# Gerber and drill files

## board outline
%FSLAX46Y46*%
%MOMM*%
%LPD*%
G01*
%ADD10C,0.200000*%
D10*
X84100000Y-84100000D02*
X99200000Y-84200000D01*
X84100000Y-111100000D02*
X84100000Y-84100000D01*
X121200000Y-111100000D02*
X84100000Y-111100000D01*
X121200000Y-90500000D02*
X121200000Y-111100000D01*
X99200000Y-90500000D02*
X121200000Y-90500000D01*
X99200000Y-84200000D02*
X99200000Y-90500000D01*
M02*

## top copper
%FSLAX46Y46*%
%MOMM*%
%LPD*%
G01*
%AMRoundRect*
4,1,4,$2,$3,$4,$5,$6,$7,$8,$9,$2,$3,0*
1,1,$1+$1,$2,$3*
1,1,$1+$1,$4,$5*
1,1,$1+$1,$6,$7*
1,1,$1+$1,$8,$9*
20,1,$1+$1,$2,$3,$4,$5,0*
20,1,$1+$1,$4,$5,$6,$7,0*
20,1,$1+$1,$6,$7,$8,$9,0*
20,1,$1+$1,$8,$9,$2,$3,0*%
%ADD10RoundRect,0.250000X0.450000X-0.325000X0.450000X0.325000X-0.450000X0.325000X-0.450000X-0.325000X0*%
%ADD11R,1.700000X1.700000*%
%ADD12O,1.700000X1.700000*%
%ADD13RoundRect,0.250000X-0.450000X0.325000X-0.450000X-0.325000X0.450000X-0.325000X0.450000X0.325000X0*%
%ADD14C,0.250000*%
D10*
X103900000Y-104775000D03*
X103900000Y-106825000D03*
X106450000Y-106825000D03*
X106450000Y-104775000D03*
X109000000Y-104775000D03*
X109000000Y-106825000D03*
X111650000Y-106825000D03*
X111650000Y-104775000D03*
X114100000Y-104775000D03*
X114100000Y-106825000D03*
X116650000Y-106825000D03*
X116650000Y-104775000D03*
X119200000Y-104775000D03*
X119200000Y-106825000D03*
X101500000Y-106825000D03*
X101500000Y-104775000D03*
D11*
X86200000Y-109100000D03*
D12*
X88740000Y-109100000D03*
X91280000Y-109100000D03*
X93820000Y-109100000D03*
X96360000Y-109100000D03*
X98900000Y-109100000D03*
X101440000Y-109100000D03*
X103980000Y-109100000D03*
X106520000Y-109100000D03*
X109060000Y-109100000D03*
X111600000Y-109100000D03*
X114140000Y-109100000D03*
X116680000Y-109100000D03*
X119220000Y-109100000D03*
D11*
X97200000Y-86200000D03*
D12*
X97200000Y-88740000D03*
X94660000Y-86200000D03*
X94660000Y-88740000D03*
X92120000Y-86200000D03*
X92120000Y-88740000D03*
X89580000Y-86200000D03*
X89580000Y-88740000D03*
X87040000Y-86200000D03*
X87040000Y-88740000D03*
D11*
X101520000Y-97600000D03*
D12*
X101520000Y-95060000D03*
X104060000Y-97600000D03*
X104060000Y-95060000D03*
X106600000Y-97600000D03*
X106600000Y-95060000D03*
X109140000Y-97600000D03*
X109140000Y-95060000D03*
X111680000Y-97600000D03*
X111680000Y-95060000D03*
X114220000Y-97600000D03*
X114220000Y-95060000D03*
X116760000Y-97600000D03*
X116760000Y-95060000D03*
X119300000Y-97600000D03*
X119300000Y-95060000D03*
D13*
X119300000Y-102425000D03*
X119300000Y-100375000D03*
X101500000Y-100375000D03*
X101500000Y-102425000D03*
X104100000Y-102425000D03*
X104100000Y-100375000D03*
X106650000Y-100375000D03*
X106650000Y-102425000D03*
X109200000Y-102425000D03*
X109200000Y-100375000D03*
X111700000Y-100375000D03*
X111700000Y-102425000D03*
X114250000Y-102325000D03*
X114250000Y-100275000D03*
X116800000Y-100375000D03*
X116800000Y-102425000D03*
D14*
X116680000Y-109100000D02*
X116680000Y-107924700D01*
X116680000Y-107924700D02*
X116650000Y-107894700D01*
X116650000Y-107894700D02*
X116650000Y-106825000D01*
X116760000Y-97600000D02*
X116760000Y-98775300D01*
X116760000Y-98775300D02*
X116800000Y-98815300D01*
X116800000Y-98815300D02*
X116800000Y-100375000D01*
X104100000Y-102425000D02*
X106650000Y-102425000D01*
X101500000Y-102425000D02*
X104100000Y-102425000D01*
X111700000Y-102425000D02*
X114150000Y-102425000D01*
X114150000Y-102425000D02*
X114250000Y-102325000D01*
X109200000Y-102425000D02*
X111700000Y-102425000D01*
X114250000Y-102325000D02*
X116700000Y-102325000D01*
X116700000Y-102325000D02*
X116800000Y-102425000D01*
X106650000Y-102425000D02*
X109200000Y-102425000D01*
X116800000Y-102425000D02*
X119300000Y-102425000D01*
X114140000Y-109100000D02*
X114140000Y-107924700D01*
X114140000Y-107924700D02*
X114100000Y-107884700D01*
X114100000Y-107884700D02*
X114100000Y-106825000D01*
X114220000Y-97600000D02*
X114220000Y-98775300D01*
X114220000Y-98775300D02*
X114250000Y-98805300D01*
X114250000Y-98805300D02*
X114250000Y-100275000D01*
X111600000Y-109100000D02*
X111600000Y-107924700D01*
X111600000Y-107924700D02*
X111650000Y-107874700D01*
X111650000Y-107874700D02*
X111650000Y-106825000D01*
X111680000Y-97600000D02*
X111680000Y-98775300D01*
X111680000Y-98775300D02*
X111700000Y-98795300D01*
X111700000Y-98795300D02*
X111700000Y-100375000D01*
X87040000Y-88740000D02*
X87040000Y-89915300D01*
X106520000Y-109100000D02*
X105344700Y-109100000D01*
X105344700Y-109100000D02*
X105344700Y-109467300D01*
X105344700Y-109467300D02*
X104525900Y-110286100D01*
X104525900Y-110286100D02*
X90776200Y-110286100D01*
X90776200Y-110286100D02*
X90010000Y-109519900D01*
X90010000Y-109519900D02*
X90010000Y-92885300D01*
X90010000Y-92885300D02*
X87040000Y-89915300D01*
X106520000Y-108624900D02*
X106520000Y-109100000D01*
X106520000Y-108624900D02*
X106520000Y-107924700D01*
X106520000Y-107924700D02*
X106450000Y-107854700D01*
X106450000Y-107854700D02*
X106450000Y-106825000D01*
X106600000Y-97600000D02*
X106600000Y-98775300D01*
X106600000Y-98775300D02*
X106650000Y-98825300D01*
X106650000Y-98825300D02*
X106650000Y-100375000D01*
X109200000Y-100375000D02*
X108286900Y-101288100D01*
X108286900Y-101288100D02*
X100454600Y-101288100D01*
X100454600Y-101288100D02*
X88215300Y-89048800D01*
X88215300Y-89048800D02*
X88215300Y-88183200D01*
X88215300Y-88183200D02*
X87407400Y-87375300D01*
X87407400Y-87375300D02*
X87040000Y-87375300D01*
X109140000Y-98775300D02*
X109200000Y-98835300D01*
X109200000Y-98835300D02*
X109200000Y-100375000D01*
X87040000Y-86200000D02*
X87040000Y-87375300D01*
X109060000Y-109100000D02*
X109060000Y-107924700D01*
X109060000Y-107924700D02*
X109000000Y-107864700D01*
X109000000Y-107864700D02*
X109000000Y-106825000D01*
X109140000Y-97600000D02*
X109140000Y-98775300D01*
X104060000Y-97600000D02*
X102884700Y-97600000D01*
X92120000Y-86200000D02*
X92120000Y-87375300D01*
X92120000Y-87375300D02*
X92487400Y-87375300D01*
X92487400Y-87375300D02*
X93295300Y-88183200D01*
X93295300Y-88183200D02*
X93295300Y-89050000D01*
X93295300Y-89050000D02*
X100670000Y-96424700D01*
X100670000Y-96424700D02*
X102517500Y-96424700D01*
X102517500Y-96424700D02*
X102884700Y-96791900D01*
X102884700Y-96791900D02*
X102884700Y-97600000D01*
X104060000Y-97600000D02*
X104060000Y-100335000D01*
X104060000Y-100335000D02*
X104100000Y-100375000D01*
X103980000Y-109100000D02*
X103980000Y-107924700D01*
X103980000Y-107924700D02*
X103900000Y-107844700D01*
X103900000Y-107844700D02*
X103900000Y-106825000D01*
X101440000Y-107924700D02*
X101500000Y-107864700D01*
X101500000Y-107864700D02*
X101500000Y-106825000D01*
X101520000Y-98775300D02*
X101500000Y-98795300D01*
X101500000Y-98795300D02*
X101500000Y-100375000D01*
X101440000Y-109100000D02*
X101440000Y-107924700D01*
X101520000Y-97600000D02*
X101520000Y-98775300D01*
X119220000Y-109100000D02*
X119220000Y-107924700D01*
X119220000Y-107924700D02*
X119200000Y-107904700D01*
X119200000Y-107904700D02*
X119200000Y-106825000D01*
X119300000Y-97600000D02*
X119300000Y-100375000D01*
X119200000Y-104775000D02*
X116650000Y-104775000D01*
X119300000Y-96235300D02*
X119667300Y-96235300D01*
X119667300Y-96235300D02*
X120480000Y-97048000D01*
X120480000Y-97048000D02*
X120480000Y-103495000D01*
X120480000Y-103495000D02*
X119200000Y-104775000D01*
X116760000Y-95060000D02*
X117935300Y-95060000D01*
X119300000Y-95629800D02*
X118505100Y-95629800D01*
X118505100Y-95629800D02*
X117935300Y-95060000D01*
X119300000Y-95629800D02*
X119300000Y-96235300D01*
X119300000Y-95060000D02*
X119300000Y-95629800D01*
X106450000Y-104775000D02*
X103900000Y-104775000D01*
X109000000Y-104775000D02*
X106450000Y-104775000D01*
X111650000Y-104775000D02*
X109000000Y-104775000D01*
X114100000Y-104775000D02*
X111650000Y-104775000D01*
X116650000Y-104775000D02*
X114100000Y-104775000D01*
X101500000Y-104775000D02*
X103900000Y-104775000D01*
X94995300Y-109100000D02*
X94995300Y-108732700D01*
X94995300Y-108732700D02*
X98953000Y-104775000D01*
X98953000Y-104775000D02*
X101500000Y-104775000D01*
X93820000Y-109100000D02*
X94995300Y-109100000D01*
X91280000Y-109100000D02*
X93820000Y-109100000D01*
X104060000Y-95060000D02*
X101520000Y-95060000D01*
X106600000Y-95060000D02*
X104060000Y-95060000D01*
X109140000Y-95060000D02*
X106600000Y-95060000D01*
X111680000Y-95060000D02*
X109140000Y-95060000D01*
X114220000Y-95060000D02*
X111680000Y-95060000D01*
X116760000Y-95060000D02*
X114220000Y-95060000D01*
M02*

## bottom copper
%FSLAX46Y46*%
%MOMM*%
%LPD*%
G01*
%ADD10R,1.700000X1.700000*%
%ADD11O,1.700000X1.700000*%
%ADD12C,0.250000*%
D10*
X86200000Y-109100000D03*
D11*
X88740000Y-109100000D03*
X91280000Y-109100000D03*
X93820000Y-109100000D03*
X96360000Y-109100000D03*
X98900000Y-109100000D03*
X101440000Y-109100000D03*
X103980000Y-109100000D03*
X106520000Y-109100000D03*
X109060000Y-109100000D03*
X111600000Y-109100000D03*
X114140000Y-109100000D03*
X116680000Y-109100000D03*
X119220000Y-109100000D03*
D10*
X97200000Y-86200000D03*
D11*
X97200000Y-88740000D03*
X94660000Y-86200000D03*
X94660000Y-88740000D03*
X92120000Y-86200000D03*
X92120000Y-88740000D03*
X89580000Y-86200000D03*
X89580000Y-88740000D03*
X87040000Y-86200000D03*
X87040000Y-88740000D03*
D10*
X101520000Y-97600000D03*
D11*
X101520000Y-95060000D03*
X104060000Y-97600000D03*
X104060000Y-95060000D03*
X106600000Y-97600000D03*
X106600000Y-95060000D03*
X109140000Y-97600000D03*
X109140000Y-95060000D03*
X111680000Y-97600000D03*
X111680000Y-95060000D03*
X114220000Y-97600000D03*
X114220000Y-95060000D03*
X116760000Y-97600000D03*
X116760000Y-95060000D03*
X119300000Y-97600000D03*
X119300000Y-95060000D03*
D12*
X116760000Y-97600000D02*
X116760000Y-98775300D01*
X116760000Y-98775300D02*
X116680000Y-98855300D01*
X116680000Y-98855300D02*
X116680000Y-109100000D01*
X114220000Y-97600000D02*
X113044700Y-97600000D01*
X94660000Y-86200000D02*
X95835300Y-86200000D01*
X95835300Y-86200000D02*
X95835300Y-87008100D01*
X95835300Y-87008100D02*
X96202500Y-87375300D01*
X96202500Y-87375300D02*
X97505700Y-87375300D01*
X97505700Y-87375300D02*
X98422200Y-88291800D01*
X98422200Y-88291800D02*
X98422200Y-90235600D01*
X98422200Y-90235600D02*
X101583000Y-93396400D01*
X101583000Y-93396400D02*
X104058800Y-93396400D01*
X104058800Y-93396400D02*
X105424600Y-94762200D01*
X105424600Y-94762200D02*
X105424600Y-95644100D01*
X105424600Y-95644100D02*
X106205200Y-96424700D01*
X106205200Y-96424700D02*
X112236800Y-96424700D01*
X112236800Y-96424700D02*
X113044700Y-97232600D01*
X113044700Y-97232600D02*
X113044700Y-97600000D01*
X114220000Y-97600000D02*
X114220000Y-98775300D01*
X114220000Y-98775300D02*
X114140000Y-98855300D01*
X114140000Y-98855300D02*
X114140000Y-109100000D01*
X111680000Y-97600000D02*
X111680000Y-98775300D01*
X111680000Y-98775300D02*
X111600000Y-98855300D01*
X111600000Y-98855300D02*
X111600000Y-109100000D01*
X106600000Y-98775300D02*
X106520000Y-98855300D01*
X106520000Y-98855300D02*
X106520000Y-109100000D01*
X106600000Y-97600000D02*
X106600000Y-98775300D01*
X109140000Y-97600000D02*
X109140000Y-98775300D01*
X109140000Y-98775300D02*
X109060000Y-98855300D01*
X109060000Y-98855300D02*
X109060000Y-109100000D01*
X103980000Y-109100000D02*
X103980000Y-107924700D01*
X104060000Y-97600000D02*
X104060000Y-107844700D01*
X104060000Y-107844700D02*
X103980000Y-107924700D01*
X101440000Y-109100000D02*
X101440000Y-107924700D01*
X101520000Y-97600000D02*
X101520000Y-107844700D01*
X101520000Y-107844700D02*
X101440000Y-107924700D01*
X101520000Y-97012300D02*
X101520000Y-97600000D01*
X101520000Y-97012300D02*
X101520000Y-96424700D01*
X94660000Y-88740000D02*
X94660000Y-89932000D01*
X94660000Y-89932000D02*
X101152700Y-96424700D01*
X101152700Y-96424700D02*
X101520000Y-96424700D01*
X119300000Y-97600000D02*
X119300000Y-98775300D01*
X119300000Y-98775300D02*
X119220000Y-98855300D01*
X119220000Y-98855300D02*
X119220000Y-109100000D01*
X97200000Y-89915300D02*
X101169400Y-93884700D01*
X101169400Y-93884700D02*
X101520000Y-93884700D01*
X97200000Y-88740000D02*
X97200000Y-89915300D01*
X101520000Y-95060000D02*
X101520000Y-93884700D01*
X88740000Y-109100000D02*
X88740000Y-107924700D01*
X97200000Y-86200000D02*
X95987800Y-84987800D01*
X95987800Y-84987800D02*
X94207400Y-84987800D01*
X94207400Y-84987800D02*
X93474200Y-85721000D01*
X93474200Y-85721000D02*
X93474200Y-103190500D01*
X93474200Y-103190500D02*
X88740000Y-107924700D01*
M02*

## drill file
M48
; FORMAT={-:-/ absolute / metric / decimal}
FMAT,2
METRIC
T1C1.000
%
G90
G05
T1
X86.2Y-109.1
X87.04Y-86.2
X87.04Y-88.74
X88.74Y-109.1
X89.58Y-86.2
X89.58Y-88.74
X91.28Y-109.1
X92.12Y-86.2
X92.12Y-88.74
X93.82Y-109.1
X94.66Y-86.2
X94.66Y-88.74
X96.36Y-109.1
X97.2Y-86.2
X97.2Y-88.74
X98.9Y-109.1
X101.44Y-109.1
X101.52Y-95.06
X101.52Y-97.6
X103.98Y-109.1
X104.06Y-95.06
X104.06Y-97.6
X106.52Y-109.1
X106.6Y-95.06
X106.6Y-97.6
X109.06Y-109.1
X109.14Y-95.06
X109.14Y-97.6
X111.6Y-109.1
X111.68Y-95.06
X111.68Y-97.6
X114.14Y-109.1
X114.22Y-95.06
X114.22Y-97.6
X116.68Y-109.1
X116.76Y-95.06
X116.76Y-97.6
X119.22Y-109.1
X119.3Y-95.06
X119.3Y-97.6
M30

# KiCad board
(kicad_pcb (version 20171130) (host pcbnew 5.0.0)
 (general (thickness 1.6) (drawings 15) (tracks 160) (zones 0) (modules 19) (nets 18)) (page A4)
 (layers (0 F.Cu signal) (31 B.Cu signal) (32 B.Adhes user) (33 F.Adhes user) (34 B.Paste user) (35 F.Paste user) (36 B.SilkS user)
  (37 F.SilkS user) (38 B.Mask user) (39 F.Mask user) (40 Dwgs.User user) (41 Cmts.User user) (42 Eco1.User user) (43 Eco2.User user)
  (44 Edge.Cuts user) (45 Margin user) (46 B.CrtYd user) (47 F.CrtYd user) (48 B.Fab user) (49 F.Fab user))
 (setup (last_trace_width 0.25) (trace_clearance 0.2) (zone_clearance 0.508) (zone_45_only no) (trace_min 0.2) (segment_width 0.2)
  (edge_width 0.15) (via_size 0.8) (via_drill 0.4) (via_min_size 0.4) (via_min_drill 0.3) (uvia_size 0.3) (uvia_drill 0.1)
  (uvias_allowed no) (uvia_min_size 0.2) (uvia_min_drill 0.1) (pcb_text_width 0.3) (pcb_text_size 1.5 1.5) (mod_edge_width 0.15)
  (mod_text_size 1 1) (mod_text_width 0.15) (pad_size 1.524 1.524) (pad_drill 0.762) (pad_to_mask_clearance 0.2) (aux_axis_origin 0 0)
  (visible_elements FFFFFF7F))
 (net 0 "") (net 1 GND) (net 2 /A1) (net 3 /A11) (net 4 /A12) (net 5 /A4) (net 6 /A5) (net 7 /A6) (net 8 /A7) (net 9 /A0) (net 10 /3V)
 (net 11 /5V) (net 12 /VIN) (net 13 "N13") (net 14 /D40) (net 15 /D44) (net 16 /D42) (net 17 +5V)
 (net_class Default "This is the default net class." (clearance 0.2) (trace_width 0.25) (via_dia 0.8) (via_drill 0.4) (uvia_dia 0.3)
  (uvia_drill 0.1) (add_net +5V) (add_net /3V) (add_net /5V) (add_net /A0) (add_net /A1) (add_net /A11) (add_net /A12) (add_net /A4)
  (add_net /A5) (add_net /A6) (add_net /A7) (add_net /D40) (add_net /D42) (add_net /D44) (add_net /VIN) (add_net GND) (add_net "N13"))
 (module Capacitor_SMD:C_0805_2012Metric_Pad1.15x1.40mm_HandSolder (layer F.Cu) (at 103.9 105.8 90)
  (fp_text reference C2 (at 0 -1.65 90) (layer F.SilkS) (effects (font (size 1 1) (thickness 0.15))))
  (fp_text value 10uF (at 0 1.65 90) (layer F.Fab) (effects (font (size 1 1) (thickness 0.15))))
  (pad 2 smd roundrect (at 1.025 0 90) (size 1.15 1.4) (layers F.Cu F.Paste F.Mask) (roundrect_rratio 0.217391) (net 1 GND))
  (pad 1 smd roundrect (at -1.025 0 90) (size 1.15 1.4) (layers F.Cu F.Paste F.Mask) (roundrect_rratio 0.217391) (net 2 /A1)))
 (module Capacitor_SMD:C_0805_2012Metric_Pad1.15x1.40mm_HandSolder (layer F.Cu) (at 106.45 105.8 90)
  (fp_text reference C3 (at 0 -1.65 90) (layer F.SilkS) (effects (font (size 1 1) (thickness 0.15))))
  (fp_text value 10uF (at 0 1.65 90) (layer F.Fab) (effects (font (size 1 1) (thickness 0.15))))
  (pad 1 smd roundrect (at -1.025 0 90) (size 1.15 1.4) (layers F.Cu F.Paste F.Mask) (roundrect_rratio 0.217391) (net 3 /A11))
  (pad 2 smd roundrect (at 1.025 0 90) (size 1.15 1.4) (layers F.Cu F.Paste F.Mask) (roundrect_rratio 0.217391) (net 1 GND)))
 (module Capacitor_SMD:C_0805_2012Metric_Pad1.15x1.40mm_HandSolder (layer F.Cu) (at 109 105.8 90)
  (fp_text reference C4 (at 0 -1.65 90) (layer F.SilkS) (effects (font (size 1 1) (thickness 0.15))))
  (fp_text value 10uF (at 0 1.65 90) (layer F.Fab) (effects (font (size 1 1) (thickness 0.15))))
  (pad 2 smd roundrect (at 1.025 0 90) (size 1.15 1.4) (layers F.Cu F.Paste F.Mask) (roundrect_rratio 0.217391) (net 1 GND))
  (pad 1 smd roundrect (at -1.025 0 90) (size 1.15 1.4) (layers F.Cu F.Paste F.Mask) (roundrect_rratio 0.217391) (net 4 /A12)))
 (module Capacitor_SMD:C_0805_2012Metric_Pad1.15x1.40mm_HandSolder (layer F.Cu) (at 111.65 105.8 90)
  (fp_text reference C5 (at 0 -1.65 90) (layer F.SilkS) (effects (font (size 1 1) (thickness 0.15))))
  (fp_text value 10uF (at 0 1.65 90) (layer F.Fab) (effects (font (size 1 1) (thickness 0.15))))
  (pad 1 smd roundrect (at -1.025 0 90) (size 1.15 1.4) (layers F.Cu F.Paste F.Mask) (roundrect_rratio 0.217391) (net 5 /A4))
  (pad 2 smd roundrect (at 1.025 0 90) (size 1.15 1.4) (layers F.Cu F.Paste F.Mask) (roundrect_rratio 0.217391) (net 1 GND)))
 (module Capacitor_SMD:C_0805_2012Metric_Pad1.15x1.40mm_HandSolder (layer F.Cu) (at 114.1 105.8 90)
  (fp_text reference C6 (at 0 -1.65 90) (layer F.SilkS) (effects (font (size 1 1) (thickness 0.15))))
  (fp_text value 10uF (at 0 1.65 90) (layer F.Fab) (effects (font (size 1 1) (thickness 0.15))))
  (pad 2 smd roundrect (at 1.025 0 90) (size 1.15 1.4) (layers F.Cu F.Paste F.Mask) (roundrect_rratio 0.217391) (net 1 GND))
  (pad 1 smd roundrect (at -1.025 0 90) (size 1.15 1.4) (layers F.Cu F.Paste F.Mask) (roundrect_rratio 0.217391) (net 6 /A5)))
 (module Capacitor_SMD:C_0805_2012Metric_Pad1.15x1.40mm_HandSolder (layer F.Cu) (at 116.65 105.8 90)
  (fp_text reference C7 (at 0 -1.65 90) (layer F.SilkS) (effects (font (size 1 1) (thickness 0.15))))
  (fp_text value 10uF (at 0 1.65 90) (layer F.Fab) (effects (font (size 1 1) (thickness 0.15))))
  (pad 1 smd roundrect (at -1.025 0 90) (size 1.15 1.4) (layers F.Cu F.Paste F.Mask) (roundrect_rratio 0.217391) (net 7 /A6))
  (pad 2 smd roundrect (at 1.025 0 90) (size 1.15 1.4) (layers F.Cu F.Paste F.Mask) (roundrect_rratio 0.217391) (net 1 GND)))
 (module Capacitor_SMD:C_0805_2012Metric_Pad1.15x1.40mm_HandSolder (layer F.Cu) (at 119.2 105.8 90)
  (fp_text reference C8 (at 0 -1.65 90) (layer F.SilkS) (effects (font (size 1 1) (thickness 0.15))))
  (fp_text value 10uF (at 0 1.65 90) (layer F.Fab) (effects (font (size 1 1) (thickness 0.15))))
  (pad 2 smd roundrect (at 1.025 0 90) (size 1.15 1.4) (layers F.Cu F.Paste F.Mask) (roundrect_rratio 0.217391) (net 1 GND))
  (pad 1 smd roundrect (at -1.025 0 90) (size 1.15 1.4) (layers F.Cu F.Paste F.Mask) (roundrect_rratio 0.217391) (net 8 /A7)))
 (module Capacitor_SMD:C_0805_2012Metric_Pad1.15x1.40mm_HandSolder (layer F.Cu) (at 101.5 105.8 90)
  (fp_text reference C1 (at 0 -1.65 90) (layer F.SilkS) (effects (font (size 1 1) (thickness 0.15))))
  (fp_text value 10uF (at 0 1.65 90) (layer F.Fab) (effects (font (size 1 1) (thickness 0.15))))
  (pad 1 smd roundrect (at -1.025 0 90) (size 1.15 1.4) (layers F.Cu F.Paste F.Mask) (roundrect_rratio 0.217391) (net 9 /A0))
  (pad 2 smd roundrect (at 1.025 0 90) (size 1.15 1.4) (layers F.Cu F.Paste F.Mask) (roundrect_rratio 0.217391) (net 1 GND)))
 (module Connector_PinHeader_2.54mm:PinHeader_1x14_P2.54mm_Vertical (layer F.Cu) (at 86.2 109.1 90)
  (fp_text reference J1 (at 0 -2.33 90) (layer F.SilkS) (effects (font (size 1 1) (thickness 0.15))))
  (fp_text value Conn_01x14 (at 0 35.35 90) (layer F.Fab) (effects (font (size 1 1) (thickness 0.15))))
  (pad 1 thru_hole rect (at 0 0 90) (size 1.7 1.7) (drill 1) (layers *.Cu *.Mask) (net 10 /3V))
  (pad 2 thru_hole oval (at 0 2.54 90) (size 1.7 1.7) (drill 1) (layers *.Cu *.Mask) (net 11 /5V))
  (pad 3 thru_hole oval (at 0 5.08 90) (size 1.7 1.7) (drill 1) (layers *.Cu *.Mask) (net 1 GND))
  (pad 4 thru_hole oval (at 0 7.62 90) (size 1.7 1.7) (drill 1) (layers *.Cu *.Mask) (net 1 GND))
  (pad 5 thru_hole oval (at 0 10.16 90) (size 1.7 1.7) (drill 1) (layers *.Cu *.Mask) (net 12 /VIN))
  (pad 6 thru_hole oval (at 0 12.7 90) (size 1.7 1.7) (drill 1) (layers *.Cu *.Mask) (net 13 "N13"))
  (pad 7 thru_hole oval (at 0 15.24 90) (size 1.7 1.7) (drill 1) (layers *.Cu *.Mask) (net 9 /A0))
  (pad 8 thru_hole oval (at 0 17.78 90) (size 1.7 1.7) (drill 1) (layers *.Cu *.Mask) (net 2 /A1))
  (pad 9 thru_hole oval (at 0 20.32 90) (size 1.7 1.7) (drill 1) (layers *.Cu *.Mask) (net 3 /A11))
  (pad 10 thru_hole oval (at 0 22.86 90) (size 1.7 1.7) (drill 1) (layers *.Cu *.Mask) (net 4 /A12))
  (pad 11 thru_hole oval (at 0 25.4 90) (size 1.7 1.7) (drill 1) (layers *.Cu *.Mask) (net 5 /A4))
  (pad 12 thru_hole oval (at 0 27.94 90) (size 1.7 1.7) (drill 1) (layers *.Cu *.Mask) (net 6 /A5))
  (pad 13 thru_hole oval (at 0 30.48 90) (size 1.7 1.7) (drill 1) (layers *.Cu *.Mask) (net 7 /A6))
  (pad 14 thru_hole oval (at 0 33.02 90) (size 1.7 1.7) (drill 1) (layers *.Cu *.Mask) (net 8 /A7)))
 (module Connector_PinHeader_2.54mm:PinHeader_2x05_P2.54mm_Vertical (layer F.Cu) (at 97.2 86.2 270)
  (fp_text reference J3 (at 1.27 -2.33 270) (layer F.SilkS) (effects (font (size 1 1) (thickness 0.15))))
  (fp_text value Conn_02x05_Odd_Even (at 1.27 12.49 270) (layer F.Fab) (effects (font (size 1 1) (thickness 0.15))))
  (pad 1 thru_hole rect (at 0 0 270) (size 1.7 1.7) (drill 1) (layers *.Cu *.Mask) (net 11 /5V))
  (pad 2 thru_hole oval (at 2.54 0 270) (size 1.7 1.7) (drill 1) (layers *.Cu *.Mask) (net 1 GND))
  (pad 3 thru_hole oval (at 0 2.54 270) (size 1.7 1.7) (drill 1) (layers *.Cu *.Mask) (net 6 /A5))
  (pad 4 thru_hole oval (at 2.54 2.54 270) (size 1.7 1.7) (drill 1) (layers *.Cu *.Mask) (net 9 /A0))
  (pad 5 thru_hole oval (at 0 5.08 270) (size 1.7 1.7) (drill 1) (layers *.Cu *.Mask) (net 2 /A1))
  (pad 6 thru_hole oval (at 2.54 5.08 270) (size 1.7 1.7) (drill 1) (layers *.Cu *.Mask) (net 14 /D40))
  (pad 7 thru_hole oval (at 0 7.62 270) (size 1.7 1.7) (drill 1) (layers *.Cu *.Mask) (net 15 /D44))
  (pad 8 thru_hole oval (at 2.54 7.62 270) (size 1.7 1.7) (drill 1) (layers *.Cu *.Mask) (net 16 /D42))
  (pad 9 thru_hole oval (at 0 10.16 270) (size 1.7 1.7) (drill 1) (layers *.Cu *.Mask) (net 4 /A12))
  (pad 10 thru_hole oval (at 2.54 10.16 270) (size 1.7 1.7) (drill 1) (layers *.Cu *.Mask) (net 3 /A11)))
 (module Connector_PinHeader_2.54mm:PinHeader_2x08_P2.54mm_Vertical (layer F.Cu) (at 101.52 97.6 90)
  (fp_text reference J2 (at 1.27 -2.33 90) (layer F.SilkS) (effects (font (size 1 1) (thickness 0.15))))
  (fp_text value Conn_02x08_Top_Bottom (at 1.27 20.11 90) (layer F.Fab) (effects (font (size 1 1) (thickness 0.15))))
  (pad 1 thru_hole rect (at 0 0 90) (size 1.7 1.7) (drill 1) (layers *.Cu *.Mask) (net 9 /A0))
  (pad 2 thru_hole oval (at 2.54 0 90) (size 1.7 1.7) (drill 1) (layers *.Cu *.Mask) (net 1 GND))
  (pad 3 thru_hole oval (at 0 2.54 90) (size 1.7 1.7) (drill 1) (layers *.Cu *.Mask) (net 2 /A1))
  (pad 4 thru_hole oval (at 2.54 2.54 90) (size 1.7 1.7) (drill 1) (layers *.Cu *.Mask) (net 1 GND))
  (pad 5 thru_hole oval (at 0 5.08 90) (size 1.7 1.7) (drill 1) (layers *.Cu *.Mask) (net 3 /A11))
  (pad 6 thru_hole oval (at 2.54 5.08 90) (size 1.7 1.7) (drill 1) (layers *.Cu *.Mask) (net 1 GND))
  (pad 7 thru_hole oval (at 0 7.62 90) (size 1.7 1.7) (drill 1) (layers *.Cu *.Mask) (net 4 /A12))
  (pad 8 thru_hole oval (at 2.54 7.62 90) (size 1.7 1.7) (drill 1) (layers *.Cu *.Mask) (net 1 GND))
  (pad 9 thru_hole oval (at 0 10.16 90) (size 1.7 1.7) (drill 1) (layers *.Cu *.Mask) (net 5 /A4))
  (pad 10 thru_hole oval (at 2.54 10.16 90) (size 1.7 1.7) (drill 1) (layers *.Cu *.Mask) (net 1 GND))
  (pad 11 thru_hole oval (at 0 12.7 90) (size 1.7 1.7) (drill 1) (layers *.Cu *.Mask) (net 6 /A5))
  (pad 12 thru_hole oval (at 2.54 12.7 90) (size 1.7 1.7) (drill 1) (layers *.Cu *.Mask) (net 1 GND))
  (pad 13 thru_hole oval (at 0 15.24 90) (size 1.7 1.7) (drill 1) (layers *.Cu *.Mask) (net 7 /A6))
  (pad 14 thru_hole oval (at 2.54 15.24 90) (size 1.7 1.7) (drill 1) (layers *.Cu *.Mask) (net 1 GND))
  (pad 15 thru_hole oval (at 0 17.78 90) (size 1.7 1.7) (drill 1) (layers *.Cu *.Mask) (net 8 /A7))
  (pad 16 thru_hole oval (at 2.54 17.78 90) (size 1.7 1.7) (drill 1) (layers *.Cu *.Mask) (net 1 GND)))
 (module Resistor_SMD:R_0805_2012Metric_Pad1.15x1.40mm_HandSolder (layer F.Cu) (at 119.3 101.4 270)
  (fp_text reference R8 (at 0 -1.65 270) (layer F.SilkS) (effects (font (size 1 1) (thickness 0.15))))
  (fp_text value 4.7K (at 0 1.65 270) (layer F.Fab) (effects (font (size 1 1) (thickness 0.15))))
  (pad 2 smd roundrect (at 1.025 0 270) (size 1.15 1.4) (layers F.Cu F.Paste F.Mask) (roundrect_rratio 0.217391) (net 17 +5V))
  (pad 1 smd roundrect (at -1.025 0 270) (size 1.15 1.4) (layers F.Cu F.Paste F.Mask) (roundrect_rratio 0.217391) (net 8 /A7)))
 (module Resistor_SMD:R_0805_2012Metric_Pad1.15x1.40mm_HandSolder (layer F.Cu) (at 101.5 101.4 270)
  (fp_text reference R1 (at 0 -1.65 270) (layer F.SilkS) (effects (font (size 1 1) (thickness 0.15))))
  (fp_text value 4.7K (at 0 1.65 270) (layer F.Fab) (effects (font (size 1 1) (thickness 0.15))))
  (pad 1 smd roundrect (at -1.025 0 270) (size 1.15 1.4) (layers F.Cu F.Paste F.Mask) (roundrect_rratio 0.217391) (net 9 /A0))
  (pad 2 smd roundrect (at 1.025 0 270) (size 1.15 1.4) (layers F.Cu F.Paste F.Mask) (roundrect_rratio 0.217391) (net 17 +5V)))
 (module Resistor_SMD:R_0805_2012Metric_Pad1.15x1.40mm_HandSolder (layer F.Cu) (at 104.1 101.4 270)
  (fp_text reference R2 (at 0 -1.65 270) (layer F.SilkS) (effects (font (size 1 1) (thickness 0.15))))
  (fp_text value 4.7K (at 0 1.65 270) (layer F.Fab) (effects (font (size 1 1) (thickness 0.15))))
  (pad 2 smd roundrect (at 1.025 0 270) (size 1.15 1.4) (layers F.Cu F.Paste F.Mask) (roundrect_rratio 0.217391) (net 17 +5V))
  (pad 1 smd roundrect (at -1.025 0 270) (size 1.15 1.4) (layers F.Cu F.Paste F.Mask) (roundrect_rratio 0.217391) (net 2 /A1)))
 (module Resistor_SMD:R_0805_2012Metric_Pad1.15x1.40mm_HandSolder (layer F.Cu) (at 106.65 101.4 270)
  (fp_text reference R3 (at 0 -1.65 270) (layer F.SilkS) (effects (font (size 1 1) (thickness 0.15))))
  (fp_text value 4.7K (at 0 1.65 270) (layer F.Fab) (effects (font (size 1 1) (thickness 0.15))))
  (pad 1 smd roundrect (at -1.025 0 270) (size 1.15 1.4) (layers F.Cu F.Paste F.Mask) (roundrect_rratio 0.217391) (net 3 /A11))
  (pad 2 smd roundrect (at 1.025 0 270) (size 1.15 1.4) (layers F.Cu F.Paste F.Mask) (roundrect_rratio 0.217391) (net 17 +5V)))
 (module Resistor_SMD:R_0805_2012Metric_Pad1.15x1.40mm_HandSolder (layer F.Cu) (at 109.2 101.4 270)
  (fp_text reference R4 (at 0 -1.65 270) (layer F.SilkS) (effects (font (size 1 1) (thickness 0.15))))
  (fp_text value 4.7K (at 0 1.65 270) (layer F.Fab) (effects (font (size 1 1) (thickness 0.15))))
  (pad 2 smd roundrect (at 1.025 0 270) (size 1.15 1.4) (layers F.Cu F.Paste F.Mask) (roundrect_rratio 0.217391) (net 17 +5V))
  (pad 1 smd roundrect (at -1.025 0 270) (size 1.15 1.4) (layers F.Cu F.Paste F.Mask) (roundrect_rratio 0.217391) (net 4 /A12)))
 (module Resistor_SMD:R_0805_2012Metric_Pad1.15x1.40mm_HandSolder (layer F.Cu) (at 111.7 101.4 270)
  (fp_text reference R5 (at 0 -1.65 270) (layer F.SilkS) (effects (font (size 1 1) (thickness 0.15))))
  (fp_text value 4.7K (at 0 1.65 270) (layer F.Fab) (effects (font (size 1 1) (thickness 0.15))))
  (pad 1 smd roundrect (at -1.025 0 270) (size 1.15 1.4) (layers F.Cu F.Paste F.Mask) (roundrect_rratio 0.217391) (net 5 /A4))
  (pad 2 smd roundrect (at 1.025 0 270) (size 1.15 1.4) (layers F.Cu F.Paste F.Mask) (roundrect_rratio 0.217391) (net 17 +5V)))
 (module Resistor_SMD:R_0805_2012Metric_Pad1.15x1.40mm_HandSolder (layer F.Cu) (at 114.25 101.3 270)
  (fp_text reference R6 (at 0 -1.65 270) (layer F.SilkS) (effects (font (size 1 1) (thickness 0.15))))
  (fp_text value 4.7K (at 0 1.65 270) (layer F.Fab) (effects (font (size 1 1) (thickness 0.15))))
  (pad 2 smd roundrect (at 1.025 0 270) (size 1.15 1.4) (layers F.Cu F.Paste F.Mask) (roundrect_rratio 0.217391) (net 17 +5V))
  (pad 1 smd roundrect (at -1.025 0 270) (size 1.15 1.4) (layers F.Cu F.Paste F.Mask) (roundrect_rratio 0.217391) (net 6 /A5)))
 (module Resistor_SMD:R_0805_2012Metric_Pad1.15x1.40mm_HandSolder (layer F.Cu) (at 116.8 101.4 270)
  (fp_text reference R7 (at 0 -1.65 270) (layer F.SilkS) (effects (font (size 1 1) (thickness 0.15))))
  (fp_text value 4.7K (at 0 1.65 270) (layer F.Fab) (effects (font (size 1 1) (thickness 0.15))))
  (pad 1 smd roundrect (at -1.025 0 270) (size 1.15 1.4) (layers F.Cu F.Paste F.Mask) (roundrect_rratio 0.217391) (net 7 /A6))
  (pad 2 smd roundrect (at 1.025 0 270) (size 1.15 1.4) (layers F.Cu F.Paste F.Mask) (roundrect_rratio 0.217391) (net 17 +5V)))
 (gr_line (start 84.1 84.1) (end 99.2 84.2) (layer Edge.Cuts) (width 0.2))
 (gr_line (start 84.1 111.1) (end 84.1 84.1) (layer Edge.Cuts) (width 0.2))
 (gr_line (start 121.2 111.1) (end 84.1 111.1) (layer Edge.Cuts) (width 0.2))
 (gr_line (start 121.2 90.5) (end 121.2 111.1) (layer Edge.Cuts) (width 0.2))
 (gr_line (start 99.2 90.5) (end 121.2 90.5) (layer Edge.Cuts) (width 0.2))
 (gr_line (start 99.2 84.2) (end 99.2 90.5) (layer Edge.Cuts) (width 0.2))
 (segment (start 116.76 97.6) (end 116.76 98.7753) (width 0.25) (layer B.Cu) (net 7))
 (segment (start 116.76 98.7753) (end 116.68 98.8553) (width 0.25) (layer B.Cu) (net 7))
 (segment (start 116.68 98.8553) (end 116.68 109.1) (width 0.25) (layer B.Cu) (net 7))
 (segment (start 116.68 109.1) (end 116.68 107.9247) (width 0.25) (layer F.Cu) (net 7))
 (segment (start 116.68 107.9247) (end 116.65 107.8947) (width 0.25) (layer F.Cu) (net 7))
 (segment (start 116.65 107.8947) (end 116.65 106.825) (width 0.25) (layer F.Cu) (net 7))
 (segment (start 116.76 97.6) (end 116.76 98.7753) (width 0.25) (layer F.Cu) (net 7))
 (segment (start 116.76 98.7753) (end 116.8 98.8153) (width 0.25) (layer F.Cu) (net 7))
 (segment (start 116.8 98.8153) (end 116.8 100.375) (width 0.25) (layer F.Cu) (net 7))
 (segment (start 104.1 102.425) (end 106.65 102.425) (width 0.25) (layer F.Cu) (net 17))
 (segment (start 101.5 102.425) (end 104.1 102.425) (width 0.25) (layer F.Cu) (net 17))
 (segment (start 111.7 102.425) (end 114.15 102.425) (width 0.25) (layer F.Cu) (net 17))
 (segment (start 114.15 102.425) (end 114.25 102.325) (width 0.25) (layer F.Cu) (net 17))
 (segment (start 109.2 102.425) (end 111.7 102.425) (width 0.25) (layer F.Cu) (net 17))
 (segment (start 114.25 102.325) (end 116.7 102.325) (width 0.25) (layer F.Cu) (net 17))
 (segment (start 116.7 102.325) (end 116.8 102.425) (width 0.25) (layer F.Cu) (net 17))
 (segment (start 106.65 102.425) (end 109.2 102.425) (width 0.25) (layer F.Cu) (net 17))
 (segment (start 116.8 102.425) (end 119.3 102.425) (width 0.25) (layer F.Cu) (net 17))
 (segment (start 114.22 97.6) (end 113.0447 97.6) (width 0.25) (layer B.Cu) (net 6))
 (segment (start 94.66 86.2) (end 95.8353 86.2) (width 0.25) (layer B.Cu) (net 6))
 (segment (start 95.8353 86.2) (end 95.8353 87.0081) (width 0.25) (layer B.Cu) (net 6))
 (segment (start 95.8353 87.0081) (end 96.2025 87.3753) (width 0.25) (layer B.Cu) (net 6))
 (segment (start 96.2025 87.3753) (end 97.5057 87.3753) (width 0.25) (layer B.Cu) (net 6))
 (segment (start 97.5057 87.3753) (end 98.4222 88.2918) (width 0.25) (layer B.Cu) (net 6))
 (segment (start 98.4222 88.2918) (end 98.4222 90.2356) (width 0.25) (layer B.Cu) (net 6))
 (segment (start 98.4222 90.2356) (end 101.583 93.3964) (width 0.25) (layer B.Cu) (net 6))
 (segment (start 101.583 93.3964) (end 104.0588 93.3964) (width 0.25) (layer B.Cu) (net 6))
 (segment (start 104.0588 93.3964) (end 105.4246 94.7622) (width 0.25) (layer B.Cu) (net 6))
 (segment (start 105.4246 94.7622) (end 105.4246 95.6441) (width 0.25) (layer B.Cu) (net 6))
 (segment (start 105.4246 95.6441) (end 106.2052 96.4247) (width 0.25) (layer B.Cu) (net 6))
 (segment (start 106.2052 96.4247) (end 112.2368 96.4247) (width 0.25) (layer B.Cu) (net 6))
 (segment (start 112.2368 96.4247) (end 113.0447 97.2326) (width 0.25) (layer B.Cu) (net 6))
 (segment (start 113.0447 97.2326) (end 113.0447 97.6) (width 0.25) (layer B.Cu) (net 6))
 (segment (start 114.22 97.6) (end 114.22 98.7753) (width 0.25) (layer B.Cu) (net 6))
 (segment (start 114.22 98.7753) (end 114.14 98.8553) (width 0.25) (layer B.Cu) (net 6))
 (segment (start 114.14 98.8553) (end 114.14 109.1) (width 0.25) (layer B.Cu) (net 6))
 (segment (start 114.14 109.1) (end 114.14 107.9247) (width 0.25) (layer F.Cu) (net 6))
 (segment (start 114.14 107.9247) (end 114.1 107.8847) (width 0.25) (layer F.Cu) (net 6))
 (segment (start 114.1 107.8847) (end 114.1 106.825) (width 0.25) (layer F.Cu) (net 6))
 (segment (start 114.22 97.6) (end 114.22 98.7753) (width 0.25) (layer F.Cu) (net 6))
 (segment (start 114.22 98.7753) (end 114.25 98.8053) (width 0.25) (layer F.Cu) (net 6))
 (segment (start 114.25 98.8053) (end 114.25 100.275) (width 0.25) (layer F.Cu) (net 6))
 (segment (start 111.68 97.6) (end 111.68 98.7753) (width 0.25) (layer B.Cu) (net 5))
 (segment (start 111.68 98.7753) (end 111.6 98.8553) (width 0.25) (layer B.Cu) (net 5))
 (segment (start 111.6 98.8553) (end 111.6 109.1) (width 0.25) (layer B.Cu) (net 5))
 (segment (start 111.6 109.1) (end 111.6 107.9247) (width 0.25) (layer F.Cu) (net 5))
 (segment (start 111.6 107.9247) (end 111.65 107.8747) (width 0.25) (layer F.Cu) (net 5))
 (segment (start 111.65 107.8747) (end 111.65 106.825) (width 0.25) (layer F.Cu) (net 5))
 (segment (start 111.68 97.6) (end 111.68 98.7753) (width 0.25) (layer F.Cu) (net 5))
 (segment (start 111.68 98.7753) (end 111.7 98.7953) (width 0.25) (layer F.Cu) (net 5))
 (segment (start 111.7 98.7953) (end 111.7 100.375) (width 0.25) (layer F.Cu) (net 5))
 (segment (start 87.04 88.74) (end 87.04 89.9153) (width 0.25) (layer F.Cu) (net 3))
 (segment (start 106.52 109.1) (end 105.3447 109.1) (width 0.25) (layer F.Cu) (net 3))
 (segment (start 105.3447 109.1) (end 105.3447 109.4673) (width 0.25) (layer F.Cu) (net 3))
 (segment (start 105.3447 109.4673) (end 104.5259 110.2861) (width 0.25) (layer F.Cu) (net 3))
 (segment (start 104.5259 110.2861) (end 90.7762 110.2861) (width 0.25) (layer F.Cu) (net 3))
 (segment (start 90.7762 110.2861) (end 90.01 109.5199) (width 0.25) (layer F.Cu) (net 3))
 (segment (start 90.01 109.5199) (end 90.01 92.8853) (width 0.25) (layer F.Cu) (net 3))
 (segment (start 90.01 92.8853) (end 87.04 89.9153) (width 0.25) (layer F.Cu) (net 3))
 (segment (start 106.52 108.6249) (end 106.52 109.1) (width 0.25) (layer F.Cu) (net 3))
 (segment (start 106.52 108.6249) (end 106.52 107.9247) (width 0.25) (layer F.Cu) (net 3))
 (segment (start 106.6 98.7753) (end 106.52 98.8553) (width 0.25) (layer B.Cu) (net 3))
 (segment (start 106.52 98.8553) (end 106.52 109.1) (width 0.25) (layer B.Cu) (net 3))
 (segment (start 106.6 97.6) (end 106.6 98.7753) (width 0.25) (layer B.Cu) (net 3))
 (segment (start 106.52 107.9247) (end 106.45 107.8547) (width 0.25) (layer F.Cu) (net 3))
 (segment (start 106.45 107.8547) (end 106.45 106.825) (width 0.25) (layer F.Cu) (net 3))
 (segment (start 106.6 97.6) (end 106.6 98.7753) (width 0.25) (layer F.Cu) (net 3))
 (segment (start 106.6 98.7753) (end 106.65 98.8253) (width 0.25) (layer F.Cu) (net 3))
 (segment (start 106.65 98.8253) (end 106.65 100.375) (width 0.25) (layer F.Cu) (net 3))
 (segment (start 109.2 100.375) (end 108.2869 101.2881) (width 0.25) (layer F.Cu) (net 4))
 (segment (start 108.2869 101.2881) (end 100.4546 101.2881) (width 0.25) (layer F.Cu) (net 4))
 (segment (start 100.4546 101.2881) (end 88.2153 89.0488) (width 0.25) (layer F.Cu) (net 4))
 (segment (start 88.2153 89.0488) (end 88.2153 88.1832) (width 0.25) (layer F.Cu) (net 4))
 (segment (start 88.2153 88.1832) (end 87.4074 87.3753) (width 0.25) (layer F.Cu) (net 4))
 (segment (start 87.4074 87.3753) (end 87.04 87.3753) (width 0.25) (layer F.Cu) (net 4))
 (segment (start 109.14 98.7753) (end 109.2 98.8353) (width 0.25) (layer F.Cu) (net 4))
 (segment (start 109.2 98.8353) (end 109.2 100.375) (width 0.25) (layer F.Cu) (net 4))
 (segment (start 87.04 86.2) (end 87.04 87.3753) (width 0.25) (layer F.Cu) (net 4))
 (segment (start 109.06 109.1) (end 109.06 107.9247) (width 0.25) (layer F.Cu) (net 4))
 (segment (start 109.06 107.9247) (end 109 107.8647) (width 0.25) (layer F.Cu) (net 4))
 (segment (start 109 107.8647) (end 109 106.825) (width 0.25) (layer F.Cu) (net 4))
 (segment (start 109.14 97.6) (end 109.14 98.7753) (width 0.25) (layer F.Cu) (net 4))
 (segment (start 109.14 97.6) (end 109.14 98.7753) (width 0.25) (layer B.Cu) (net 4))
 (segment (start 109.14 98.7753) (end 109.06 98.8553) (width 0.25) (layer B.Cu) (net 4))
 (segment (start 109.06 98.8553) (end 109.06 109.1) (width 0.25) (layer B.Cu) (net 4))
 (segment (start 103.98 109.1) (end 103.98 107.9247) (width 0.25) (layer B.Cu) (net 2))
 (segment (start 104.06 97.6) (end 104.06 107.8447) (width 0.25) (layer B.Cu) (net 2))
 (segment (start 104.06 107.8447) (end 103.98 107.9247) (width 0.25) (layer B.Cu) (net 2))
 (segment (start 104.06 97.6) (end 102.8847 97.6) (width 0.25) (layer F.Cu) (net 2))
 (segment (start 92.12 86.2) (end 92.12 87.3753) (width 0.25) (layer F.Cu) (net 2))
 (segment (start 92.12 87.3753) (end 92.4874 87.3753) (width 0.25) (layer F.Cu) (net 2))
 (segment (start 92.4874 87.3753) (end 93.2953 88.1832) (width 0.25) (layer F.Cu) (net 2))
 (segment (start 93.2953 88.1832) (end 93.2953 89.05) (width 0.25) (layer F.Cu) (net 2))
 (segment (start 93.2953 89.05) (end 100.67 96.4247) (width 0.25) (layer F.Cu) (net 2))
 (segment (start 100.67 96.4247) (end 102.5175 96.4247) (width 0.25) (layer F.Cu) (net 2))
 (segment (start 102.5175 96.4247) (end 102.8847 96.7919) (width 0.25) (layer F.Cu) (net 2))
 (segment (start 102.8847 96.7919) (end 102.8847 97.6) (width 0.25) (layer F.Cu) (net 2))
 (segment (start 104.06 97.6) (end 104.06 100.335) (width 0.25) (layer F.Cu) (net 2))
 (segment (start 104.06 100.335) (end 104.1 100.375) (width 0.25) (layer F.Cu) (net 2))
 (segment (start 103.98 109.1) (end 103.98 107.9247) (width 0.25) (layer F.Cu) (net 2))
 (segment (start 103.98 107.9247) (end 103.9 107.8447) (width 0.25) (layer F.Cu) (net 2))
 (segment (start 103.9 107.8447) (end 103.9 106.825) (width 0.25) (layer F.Cu) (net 2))
 (segment (start 101.44 109.1) (end 101.44 107.9247) (width 0.25) (layer B.Cu) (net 9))
 (segment (start 101.52 97.6) (end 101.52 107.8447) (width 0.25) (layer B.Cu) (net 9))
 (segment (start 101.52 107.8447) (end 101.44 107.9247) (width 0.25) (layer B.Cu) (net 9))
 (segment (start 101.52 97.0123) (end 101.52 97.6) (width 0.25) (layer B.Cu) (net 9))
 (segment (start 101.52 97.0123) (end 101.52 96.4247) (width 0.25) (layer B.Cu) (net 9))
 (segment (start 101.44 107.9247) (end 101.5 107.8647) (width 0.25) (layer F.Cu) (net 9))
 (segment (start 101.5 107.8647) (end 101.5 106.825) (width 0.25) (layer F.Cu) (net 9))
 (segment (start 101.52 98.7753) (end 101.5 98.7953) (width 0.25) (layer F.Cu) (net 9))
 (segment (start 101.5 98.7953) (end 101.5 100.375) (width 0.25) (layer F.Cu) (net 9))
 (segment (start 101.44 109.1) (end 101.44 107.9247) (width 0.25) (layer F.Cu) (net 9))
 (segment (start 94.66 88.74) (end 94.66 89.932) (width 0.25) (layer B.Cu) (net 9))
 (segment (start 94.66 89.932) (end 101.1527 96.4247) (width 0.25) (layer B.Cu) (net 9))
 (segment (start 101.1527 96.4247) (end 101.52 96.4247) (width 0.25) (layer B.Cu) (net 9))
 (segment (start 101.52 97.6) (end 101.52 98.7753) (width 0.25) (layer F.Cu) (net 9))
 (segment (start 119.3 97.6) (end 119.3 98.7753) (width 0.25) (layer B.Cu) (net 8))
 (segment (start 119.3 98.7753) (end 119.22 98.8553) (width 0.25) (layer B.Cu) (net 8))
 (segment (start 119.22 98.8553) (end 119.22 109.1) (width 0.25) (layer B.Cu) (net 8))
 (segment (start 119.22 109.1) (end 119.22 107.9247) (width 0.25) (layer F.Cu) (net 8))
 (segment (start 119.22 107.9247) (end 119.2 107.9047) (width 0.25) (layer F.Cu) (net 8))
 (segment (start 119.2 107.9047) (end 119.2 106.825) (width 0.25) (layer F.Cu) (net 8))
 (segment (start 119.3 97.6) (end 119.3 100.375) (width 0.25) (layer F.Cu) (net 8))
 (segment (start 119.2 104.775) (end 116.65 104.775) (width 0.25) (layer F.Cu) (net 1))
 (segment (start 119.3 96.2353) (end 119.6673 96.2353) (width 0.25) (layer F.Cu) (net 1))
 (segment (start 119.6673 96.2353) (end 120.48 97.048) (width 0.25) (layer F.Cu) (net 1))
 (segment (start 120.48 97.048) (end 120.48 103.495) (width 0.25) (layer F.Cu) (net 1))
 (segment (start 120.48 103.495) (end 119.2 104.775) (width 0.25) (layer F.Cu) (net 1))
 (segment (start 116.76 95.06) (end 117.9353 95.06) (width 0.25) (layer F.Cu) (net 1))
 (segment (start 119.3 95.6298) (end 118.5051 95.6298) (width 0.25) (layer F.Cu) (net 1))
 (segment (start 118.5051 95.6298) (end 117.9353 95.06) (width 0.25) (layer F.Cu) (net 1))
 (segment (start 119.3 95.6298) (end 119.3 96.2353) (width 0.25) (layer F.Cu) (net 1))
 (segment (start 119.3 95.06) (end 119.3 95.6298) (width 0.25) (layer F.Cu) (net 1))
 (segment (start 106.45 104.775) (end 103.9 104.775) (width 0.25) (layer F.Cu) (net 1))
 (segment (start 109 104.775) (end 106.45 104.775) (width 0.25) (layer F.Cu) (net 1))
 (segment (start 111.65 104.775) (end 109 104.775) (width 0.25) (layer F.Cu) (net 1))
 (segment (start 114.1 104.775) (end 111.65 104.775) (width 0.25) (layer F.Cu) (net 1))
 (segment (start 116.65 104.775) (end 114.1 104.775) (width 0.25) (layer F.Cu) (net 1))
 (segment (start 101.5 104.775) (end 103.9 104.775) (width 0.25) (layer F.Cu) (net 1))
 (segment (start 94.9953 109.1) (end 94.9953 108.7327) (width 0.25) (layer F.Cu) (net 1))
 (segment (start 94.9953 108.7327) (end 98.953 104.775) (width 0.25) (layer F.Cu) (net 1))
 (segment (start 98.953 104.775) (end 101.5 104.775) (width 0.25) (layer F.Cu) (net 1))
 (segment (start 93.82 109.1) (end 94.9953 109.1) (width 0.25) (layer F.Cu) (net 1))
 (segment (start 91.28 109.1) (end 93.82 109.1) (width 0.25) (layer F.Cu) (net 1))
 (segment (start 97.2 89.9153) (end 101.1694 93.8847) (width 0.25) (layer B.Cu) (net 1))
 (segment (start 101.1694 93.8847) (end 101.52 93.8847) (width 0.25) (layer B.Cu) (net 1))
 (segment (start 97.2 88.74) (end 97.2 89.9153) (width 0.25) (layer B.Cu) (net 1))
 (segment (start 101.52 95.06) (end 101.52 93.8847) (width 0.25) (layer B.Cu) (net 1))
 (segment (start 104.06 95.06) (end 101.52 95.06) (width 0.25) (layer F.Cu) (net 1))
 (segment (start 106.6 95.06) (end 104.06 95.06) (width 0.25) (layer F.Cu) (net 1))
 (segment (start 109.14 95.06) (end 106.6 95.06) (width 0.25) (layer F.Cu) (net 1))
 (segment (start 111.68 95.06) (end 109.14 95.06) (width 0.25) (layer F.Cu) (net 1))
 (segment (start 114.22 95.06) (end 111.68 95.06) (width 0.25) (layer F.Cu) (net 1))
 (segment (start 116.76 95.06) (end 114.22 95.06) (width 0.25) (layer F.Cu) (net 1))
 (segment (start 88.74 109.1) (end 88.74 107.9247) (width 0.25) (layer B.Cu) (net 11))
 (segment (start 97.2 86.2) (end 95.9878 84.9878) (width 0.25) (layer B.Cu) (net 11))
 (segment (start 95.9878 84.9878) (end 94.2074 84.9878) (width 0.25) (layer B.Cu) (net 11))
 (segment (start 94.2074 84.9878) (end 93.4742 85.721) (width 0.25) (layer B.Cu) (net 11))
 (segment (start 93.4742 85.721) (end 93.4742 103.1905) (width 0.25) (layer B.Cu) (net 11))
 (segment (start 93.4742 103.1905) (end 88.74 107.9247) (width 0.25) (layer B.Cu) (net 11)))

